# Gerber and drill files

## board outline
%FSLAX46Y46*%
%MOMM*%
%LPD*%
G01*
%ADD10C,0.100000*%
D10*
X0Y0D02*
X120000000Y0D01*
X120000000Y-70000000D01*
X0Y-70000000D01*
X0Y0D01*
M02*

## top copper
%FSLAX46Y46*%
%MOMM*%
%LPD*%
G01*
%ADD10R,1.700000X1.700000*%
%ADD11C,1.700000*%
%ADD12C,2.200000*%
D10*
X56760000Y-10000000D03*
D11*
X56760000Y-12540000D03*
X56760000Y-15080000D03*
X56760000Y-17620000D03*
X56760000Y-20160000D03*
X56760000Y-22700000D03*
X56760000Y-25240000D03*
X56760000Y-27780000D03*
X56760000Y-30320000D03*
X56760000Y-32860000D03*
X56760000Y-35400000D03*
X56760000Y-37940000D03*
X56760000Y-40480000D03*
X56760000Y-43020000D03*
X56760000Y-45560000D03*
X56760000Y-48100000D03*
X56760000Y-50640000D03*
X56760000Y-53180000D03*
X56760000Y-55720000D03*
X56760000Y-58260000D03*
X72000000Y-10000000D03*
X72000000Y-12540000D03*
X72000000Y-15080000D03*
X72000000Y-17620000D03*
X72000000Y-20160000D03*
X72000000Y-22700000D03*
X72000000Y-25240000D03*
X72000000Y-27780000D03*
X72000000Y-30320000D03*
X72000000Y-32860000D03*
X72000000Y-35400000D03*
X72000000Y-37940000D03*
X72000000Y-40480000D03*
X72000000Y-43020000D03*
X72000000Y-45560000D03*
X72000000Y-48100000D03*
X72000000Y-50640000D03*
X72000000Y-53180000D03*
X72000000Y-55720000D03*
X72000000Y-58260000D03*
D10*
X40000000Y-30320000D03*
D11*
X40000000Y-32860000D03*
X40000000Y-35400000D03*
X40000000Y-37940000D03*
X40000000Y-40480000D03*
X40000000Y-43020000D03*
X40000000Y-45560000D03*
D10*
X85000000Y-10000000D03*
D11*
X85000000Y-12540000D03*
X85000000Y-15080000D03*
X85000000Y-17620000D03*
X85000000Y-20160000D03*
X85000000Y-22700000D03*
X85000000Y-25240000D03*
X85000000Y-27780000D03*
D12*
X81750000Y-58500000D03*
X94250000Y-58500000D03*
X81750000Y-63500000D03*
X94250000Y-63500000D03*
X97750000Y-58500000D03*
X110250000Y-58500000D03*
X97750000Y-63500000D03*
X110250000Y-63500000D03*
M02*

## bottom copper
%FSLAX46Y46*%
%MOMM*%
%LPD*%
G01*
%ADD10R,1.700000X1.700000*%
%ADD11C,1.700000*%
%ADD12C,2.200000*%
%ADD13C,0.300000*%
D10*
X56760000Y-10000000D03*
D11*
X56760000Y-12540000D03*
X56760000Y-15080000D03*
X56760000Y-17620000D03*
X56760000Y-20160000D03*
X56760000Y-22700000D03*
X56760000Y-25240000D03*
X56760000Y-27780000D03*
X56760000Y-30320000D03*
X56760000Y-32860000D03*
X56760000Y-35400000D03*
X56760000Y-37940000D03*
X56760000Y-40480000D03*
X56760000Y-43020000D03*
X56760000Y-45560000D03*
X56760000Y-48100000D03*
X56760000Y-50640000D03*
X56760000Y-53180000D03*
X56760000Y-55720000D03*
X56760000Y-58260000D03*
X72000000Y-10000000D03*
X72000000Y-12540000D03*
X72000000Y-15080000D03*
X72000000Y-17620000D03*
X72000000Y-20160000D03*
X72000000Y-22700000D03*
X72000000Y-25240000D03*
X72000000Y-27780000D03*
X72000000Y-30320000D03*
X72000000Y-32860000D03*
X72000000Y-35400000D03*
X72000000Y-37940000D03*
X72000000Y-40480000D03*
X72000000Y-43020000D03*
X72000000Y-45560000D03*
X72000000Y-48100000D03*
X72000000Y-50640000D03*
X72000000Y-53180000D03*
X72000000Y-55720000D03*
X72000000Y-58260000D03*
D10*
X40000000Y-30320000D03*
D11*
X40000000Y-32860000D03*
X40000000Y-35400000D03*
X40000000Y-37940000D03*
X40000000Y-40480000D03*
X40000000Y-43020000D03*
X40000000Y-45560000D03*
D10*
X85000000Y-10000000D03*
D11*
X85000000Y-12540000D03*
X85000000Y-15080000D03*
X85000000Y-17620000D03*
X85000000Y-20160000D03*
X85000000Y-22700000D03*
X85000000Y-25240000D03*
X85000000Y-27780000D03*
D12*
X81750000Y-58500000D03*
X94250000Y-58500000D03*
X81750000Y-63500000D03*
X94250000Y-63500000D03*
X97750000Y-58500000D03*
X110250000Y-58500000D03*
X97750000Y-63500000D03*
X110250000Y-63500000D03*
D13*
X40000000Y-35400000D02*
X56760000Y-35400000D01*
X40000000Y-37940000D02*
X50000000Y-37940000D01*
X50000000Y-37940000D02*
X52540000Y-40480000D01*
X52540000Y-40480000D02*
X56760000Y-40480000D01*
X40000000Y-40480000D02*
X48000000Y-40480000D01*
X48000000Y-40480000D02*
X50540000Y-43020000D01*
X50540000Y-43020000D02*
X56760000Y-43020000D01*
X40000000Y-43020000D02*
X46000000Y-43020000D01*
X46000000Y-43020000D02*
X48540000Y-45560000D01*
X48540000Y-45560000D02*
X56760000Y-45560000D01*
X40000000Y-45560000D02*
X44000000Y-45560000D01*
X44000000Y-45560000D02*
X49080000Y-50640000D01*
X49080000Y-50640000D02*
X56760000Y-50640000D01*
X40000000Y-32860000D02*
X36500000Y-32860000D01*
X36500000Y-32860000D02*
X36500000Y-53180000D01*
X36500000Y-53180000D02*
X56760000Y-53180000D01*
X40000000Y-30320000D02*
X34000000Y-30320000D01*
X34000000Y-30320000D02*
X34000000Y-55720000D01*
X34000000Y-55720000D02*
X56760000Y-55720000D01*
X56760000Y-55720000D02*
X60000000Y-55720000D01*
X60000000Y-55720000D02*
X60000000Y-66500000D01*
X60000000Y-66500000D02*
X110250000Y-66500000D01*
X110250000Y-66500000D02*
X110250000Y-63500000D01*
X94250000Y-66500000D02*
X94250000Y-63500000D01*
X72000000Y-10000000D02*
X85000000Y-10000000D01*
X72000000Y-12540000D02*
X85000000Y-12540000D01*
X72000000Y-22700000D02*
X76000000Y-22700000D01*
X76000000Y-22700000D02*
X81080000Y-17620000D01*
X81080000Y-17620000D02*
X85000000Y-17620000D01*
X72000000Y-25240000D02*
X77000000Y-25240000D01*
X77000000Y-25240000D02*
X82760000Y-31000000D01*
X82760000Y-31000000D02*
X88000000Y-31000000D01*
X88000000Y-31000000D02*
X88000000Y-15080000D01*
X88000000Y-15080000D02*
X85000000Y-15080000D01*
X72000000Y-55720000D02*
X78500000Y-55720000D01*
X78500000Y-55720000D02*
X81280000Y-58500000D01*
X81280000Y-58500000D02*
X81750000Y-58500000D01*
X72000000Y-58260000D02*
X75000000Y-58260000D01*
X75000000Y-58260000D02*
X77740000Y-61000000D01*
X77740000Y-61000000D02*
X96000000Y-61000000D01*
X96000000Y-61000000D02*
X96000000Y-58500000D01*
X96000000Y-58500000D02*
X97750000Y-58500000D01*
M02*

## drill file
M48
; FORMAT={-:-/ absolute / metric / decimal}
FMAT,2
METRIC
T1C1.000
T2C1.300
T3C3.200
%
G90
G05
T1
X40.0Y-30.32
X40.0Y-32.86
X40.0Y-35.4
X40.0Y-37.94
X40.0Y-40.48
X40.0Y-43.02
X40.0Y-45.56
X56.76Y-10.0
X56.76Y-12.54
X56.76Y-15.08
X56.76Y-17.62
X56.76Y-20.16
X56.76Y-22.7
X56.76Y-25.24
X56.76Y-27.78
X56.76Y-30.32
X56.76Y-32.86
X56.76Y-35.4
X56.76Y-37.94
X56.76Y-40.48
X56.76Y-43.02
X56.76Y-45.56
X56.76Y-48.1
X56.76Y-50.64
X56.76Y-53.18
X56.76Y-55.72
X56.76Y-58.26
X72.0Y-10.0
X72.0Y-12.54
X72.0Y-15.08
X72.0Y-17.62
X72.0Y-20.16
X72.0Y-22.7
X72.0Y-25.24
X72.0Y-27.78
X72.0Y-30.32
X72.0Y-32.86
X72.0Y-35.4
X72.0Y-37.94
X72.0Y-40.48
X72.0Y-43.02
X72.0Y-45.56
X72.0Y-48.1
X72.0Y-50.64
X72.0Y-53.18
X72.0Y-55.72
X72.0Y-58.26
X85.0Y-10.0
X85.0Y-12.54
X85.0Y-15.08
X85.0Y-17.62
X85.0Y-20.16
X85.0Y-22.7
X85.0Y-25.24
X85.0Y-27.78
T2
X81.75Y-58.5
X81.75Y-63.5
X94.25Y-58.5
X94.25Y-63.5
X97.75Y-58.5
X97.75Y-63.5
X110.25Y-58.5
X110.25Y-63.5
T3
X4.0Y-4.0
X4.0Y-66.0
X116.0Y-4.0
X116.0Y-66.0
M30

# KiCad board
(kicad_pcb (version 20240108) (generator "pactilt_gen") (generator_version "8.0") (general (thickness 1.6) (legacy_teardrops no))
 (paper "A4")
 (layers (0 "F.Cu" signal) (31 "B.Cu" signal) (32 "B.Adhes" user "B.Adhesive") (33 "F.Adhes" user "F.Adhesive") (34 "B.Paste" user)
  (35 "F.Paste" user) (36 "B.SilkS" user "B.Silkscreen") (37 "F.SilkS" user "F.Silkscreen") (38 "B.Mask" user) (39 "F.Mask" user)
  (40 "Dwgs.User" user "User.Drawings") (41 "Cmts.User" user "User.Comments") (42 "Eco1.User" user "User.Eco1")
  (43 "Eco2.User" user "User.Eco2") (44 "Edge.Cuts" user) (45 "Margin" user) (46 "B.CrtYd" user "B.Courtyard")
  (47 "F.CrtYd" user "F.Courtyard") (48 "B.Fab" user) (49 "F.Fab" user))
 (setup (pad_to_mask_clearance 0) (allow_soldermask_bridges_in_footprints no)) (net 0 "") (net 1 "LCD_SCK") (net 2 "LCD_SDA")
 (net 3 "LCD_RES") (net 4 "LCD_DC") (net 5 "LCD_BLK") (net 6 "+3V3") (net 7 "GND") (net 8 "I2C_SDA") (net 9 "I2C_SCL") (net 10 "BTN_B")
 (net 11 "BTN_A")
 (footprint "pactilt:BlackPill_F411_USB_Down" (layer "F.Cu") (at 56.76 10)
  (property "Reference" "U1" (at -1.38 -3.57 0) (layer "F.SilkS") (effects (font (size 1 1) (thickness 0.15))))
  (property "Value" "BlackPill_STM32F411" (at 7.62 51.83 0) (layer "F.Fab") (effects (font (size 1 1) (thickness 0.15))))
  (pad "1" thru_hole rect (at 0 0) (size 1.7 1.7) (drill 1.0) (layers "*.Cu" "*.Mask"))
  (pad "2" thru_hole circle (at 0 2.54) (size 1.7 1.7) (drill 1.0) (layers "*.Cu" "*.Mask"))
  (pad "3" thru_hole circle (at 0 5.08) (size 1.7 1.7) (drill 1.0) (layers "*.Cu" "*.Mask"))
  (pad "4" thru_hole circle (at 0 7.62) (size 1.7 1.7) (drill 1.0) (layers "*.Cu" "*.Mask"))
  (pad "5" thru_hole circle (at 0 10.16) (size 1.7 1.7) (drill 1.0) (layers "*.Cu" "*.Mask"))
  (pad "6" thru_hole circle (at 0 12.7) (size 1.7 1.7) (drill 1.0) (layers "*.Cu" "*.Mask"))
  (pad "7" thru_hole circle (at 0 15.24) (size 1.7 1.7) (drill 1.0) (layers "*.Cu" "*.Mask"))
  (pad "8" thru_hole circle (at 0 17.78) (size 1.7 1.7) (drill 1.0) (layers "*.Cu" "*.Mask"))
  (pad "9" thru_hole circle (at 0 20.32) (size 1.7 1.7) (drill 1.0) (layers "*.Cu" "*.Mask"))
  (pad "10" thru_hole circle (at 0 22.86) (size 1.7 1.7) (drill 1.0) (layers "*.Cu" "*.Mask"))
  (pad "11" thru_hole circle (at 0 25.4) (size 1.7 1.7) (drill 1.0) (layers "*.Cu" "*.Mask") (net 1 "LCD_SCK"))
  (pad "12" thru_hole circle (at 0 27.94) (size 1.7 1.7) (drill 1.0) (layers "*.Cu" "*.Mask"))
  (pad "13" thru_hole circle (at 0 30.48) (size 1.7 1.7) (drill 1.0) (layers "*.Cu" "*.Mask") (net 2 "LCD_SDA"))
  (pad "14" thru_hole circle (at 0 33.02) (size 1.7 1.7) (drill 1.0) (layers "*.Cu" "*.Mask") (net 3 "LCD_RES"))
  (pad "15" thru_hole circle (at 0 35.56) (size 1.7 1.7) (drill 1.0) (layers "*.Cu" "*.Mask") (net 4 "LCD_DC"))
  (pad "16" thru_hole circle (at 0 38.1) (size 1.7 1.7) (drill 1.0) (layers "*.Cu" "*.Mask"))
  (pad "17" thru_hole circle (at 0 40.64) (size 1.7 1.7) (drill 1.0) (layers "*.Cu" "*.Mask") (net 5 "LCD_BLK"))
  (pad "18" thru_hole circle (at 0 43.18) (size 1.7 1.7) (drill 1.0) (layers "*.Cu" "*.Mask") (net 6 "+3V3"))
  (pad "19" thru_hole circle (at 0 45.72) (size 1.7 1.7) (drill 1.0) (layers "*.Cu" "*.Mask") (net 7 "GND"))
  (pad "20" thru_hole circle (at 0 48.26) (size 1.7 1.7) (drill 1.0) (layers "*.Cu" "*.Mask"))
  (pad "21" thru_hole circle (at 15.24 0) (size 1.7 1.7) (drill 1.0) (layers "*.Cu" "*.Mask") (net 6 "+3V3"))
  (pad "22" thru_hole circle (at 15.24 2.54) (size 1.7 1.7) (drill 1.0) (layers "*.Cu" "*.Mask") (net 7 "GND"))
  (pad "23" thru_hole circle (at 15.24 5.08) (size 1.7 1.7) (drill 1.0) (layers "*.Cu" "*.Mask"))
  (pad "24" thru_hole circle (at 15.24 7.62) (size 1.7 1.7) (drill 1.0) (layers "*.Cu" "*.Mask"))
  (pad "25" thru_hole circle (at 15.24 10.16) (size 1.7 1.7) (drill 1.0) (layers "*.Cu" "*.Mask"))
  (pad "26" thru_hole circle (at 15.24 12.7) (size 1.7 1.7) (drill 1.0) (layers "*.Cu" "*.Mask") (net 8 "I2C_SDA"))
  (pad "27" thru_hole circle (at 15.24 15.24) (size 1.7 1.7) (drill 1.0) (layers "*.Cu" "*.Mask") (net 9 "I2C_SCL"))
  (pad "28" thru_hole circle (at 15.24 17.78) (size 1.7 1.7) (drill 1.0) (layers "*.Cu" "*.Mask"))
  (pad "29" thru_hole circle (at 15.24 20.32) (size 1.7 1.7) (drill 1.0) (layers "*.Cu" "*.Mask"))
  (pad "30" thru_hole circle (at 15.24 22.86) (size 1.7 1.7) (drill 1.0) (layers "*.Cu" "*.Mask"))
  (pad "31" thru_hole circle (at 15.24 25.4) (size 1.7 1.7) (drill 1.0) (layers "*.Cu" "*.Mask"))
  (pad "32" thru_hole circle (at 15.24 27.94) (size 1.7 1.7) (drill 1.0) (layers "*.Cu" "*.Mask"))
  (pad "33" thru_hole circle (at 15.24 30.48) (size 1.7 1.7) (drill 1.0) (layers "*.Cu" "*.Mask"))
  (pad "34" thru_hole circle (at 15.24 33.02) (size 1.7 1.7) (drill 1.0) (layers "*.Cu" "*.Mask"))
  (pad "35" thru_hole circle (at 15.24 35.56) (size 1.7 1.7) (drill 1.0) (layers "*.Cu" "*.Mask"))
  (pad "36" thru_hole circle (at 15.24 38.1) (size 1.7 1.7) (drill 1.0) (layers "*.Cu" "*.Mask"))
  (pad "37" thru_hole circle (at 15.24 40.64) (size 1.7 1.7) (drill 1.0) (layers "*.Cu" "*.Mask"))
  (pad "38" thru_hole circle (at 15.24 43.18) (size 1.7 1.7) (drill 1.0) (layers "*.Cu" "*.Mask"))
  (pad "39" thru_hole circle (at 15.24 45.72) (size 1.7 1.7) (drill 1.0) (layers "*.Cu" "*.Mask") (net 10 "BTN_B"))
  (pad "40" thru_hole circle (at 15.24 48.26) (size 1.7 1.7) (drill 1.0) (layers "*.Cu" "*.Mask") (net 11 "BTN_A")))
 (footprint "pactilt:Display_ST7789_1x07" (layer "F.Cu") (at 40 30.32)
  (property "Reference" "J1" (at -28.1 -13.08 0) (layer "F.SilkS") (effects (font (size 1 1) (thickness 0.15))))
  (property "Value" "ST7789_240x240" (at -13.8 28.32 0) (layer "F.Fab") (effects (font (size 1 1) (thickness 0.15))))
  (pad "1" thru_hole rect (at 0 0) (size 1.7 1.7) (drill 1.0) (layers "*.Cu" "*.Mask") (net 7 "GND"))
  (pad "2" thru_hole circle (at 0 2.54) (size 1.7 1.7) (drill 1.0) (layers "*.Cu" "*.Mask") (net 6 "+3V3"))
  (pad "3" thru_hole circle (at 0 5.08) (size 1.7 1.7) (drill 1.0) (layers "*.Cu" "*.Mask") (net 1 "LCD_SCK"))
  (pad "4" thru_hole circle (at 0 7.62) (size 1.7 1.7) (drill 1.0) (layers "*.Cu" "*.Mask") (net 2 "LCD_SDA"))
  (pad "5" thru_hole circle (at 0 10.16) (size 1.7 1.7) (drill 1.0) (layers "*.Cu" "*.Mask") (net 3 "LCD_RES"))
  (pad "6" thru_hole circle (at 0 12.7) (size 1.7 1.7) (drill 1.0) (layers "*.Cu" "*.Mask") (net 4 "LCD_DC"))
  (pad "7" thru_hole circle (at 0 15.24) (size 1.7 1.7) (drill 1.0) (layers "*.Cu" "*.Mask") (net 5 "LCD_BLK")))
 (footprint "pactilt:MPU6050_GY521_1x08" (layer "F.Cu") (at 85 10)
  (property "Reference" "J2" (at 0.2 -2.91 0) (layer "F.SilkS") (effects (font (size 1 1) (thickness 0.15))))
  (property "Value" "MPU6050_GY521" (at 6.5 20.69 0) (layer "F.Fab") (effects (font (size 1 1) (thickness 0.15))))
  (pad "1" thru_hole rect (at 0 0) (size 1.7 1.7) (drill 1.0) (layers "*.Cu" "*.Mask") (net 6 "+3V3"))
  (pad "2" thru_hole circle (at 0 2.54) (size 1.7 1.7) (drill 1.0) (layers "*.Cu" "*.Mask") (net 7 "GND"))
  (pad "3" thru_hole circle (at 0 5.08) (size 1.7 1.7) (drill 1.0) (layers "*.Cu" "*.Mask") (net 9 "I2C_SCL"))
  (pad "4" thru_hole circle (at 0 7.62) (size 1.7 1.7) (drill 1.0) (layers "*.Cu" "*.Mask") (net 8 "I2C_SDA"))
  (pad "5" thru_hole circle (at 0 10.16) (size 1.7 1.7) (drill 1.0) (layers "*.Cu" "*.Mask"))
  (pad "6" thru_hole circle (at 0 12.7) (size 1.7 1.7) (drill 1.0) (layers "*.Cu" "*.Mask"))
  (pad "7" thru_hole circle (at 0 15.24) (size 1.7 1.7) (drill 1.0) (layers "*.Cu" "*.Mask"))
  (pad "8" thru_hole circle (at 0 17.78) (size 1.7 1.7) (drill 1.0) (layers "*.Cu" "*.Mask")))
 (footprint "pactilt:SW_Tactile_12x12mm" (layer "F.Cu") (at 81.75 58.5)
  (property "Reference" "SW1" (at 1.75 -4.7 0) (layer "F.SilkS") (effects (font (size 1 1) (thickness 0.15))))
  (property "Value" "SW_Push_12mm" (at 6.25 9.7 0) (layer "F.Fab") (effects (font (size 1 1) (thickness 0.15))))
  (pad "1" thru_hole circle (at 0 0) (size 2.2 2.2) (drill 1.3) (layers "*.Cu" "*.Mask") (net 10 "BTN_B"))
  (pad "2" thru_hole circle (at 12.5 0) (size 2.2 2.2) (drill 1.3) (layers "*.Cu" "*.Mask"))
  (pad "3" thru_hole circle (at 0 5) (size 2.2 2.2) (drill 1.3) (layers "*.Cu" "*.Mask"))
  (pad "4" thru_hole circle (at 12.5 5) (size 2.2 2.2) (drill 1.3) (layers "*.Cu" "*.Mask") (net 7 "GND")))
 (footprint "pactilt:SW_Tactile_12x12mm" (layer "F.Cu") (at 97.75 58.5)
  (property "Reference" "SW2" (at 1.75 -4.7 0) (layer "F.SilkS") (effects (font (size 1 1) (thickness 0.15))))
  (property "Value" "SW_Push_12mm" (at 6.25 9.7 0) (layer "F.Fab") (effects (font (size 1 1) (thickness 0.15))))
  (pad "1" thru_hole circle (at 0 0) (size 2.2 2.2) (drill 1.3) (layers "*.Cu" "*.Mask") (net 11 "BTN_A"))
  (pad "2" thru_hole circle (at 12.5 0) (size 2.2 2.2) (drill 1.3) (layers "*.Cu" "*.Mask"))
  (pad "3" thru_hole circle (at 0 5) (size 2.2 2.2) (drill 1.3) (layers "*.Cu" "*.Mask"))
  (pad "4" thru_hole circle (at 12.5 5) (size 2.2 2.2) (drill 1.3) (layers "*.Cu" "*.Mask") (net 7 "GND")))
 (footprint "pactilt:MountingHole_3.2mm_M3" (layer "F.Cu") (at 4 4)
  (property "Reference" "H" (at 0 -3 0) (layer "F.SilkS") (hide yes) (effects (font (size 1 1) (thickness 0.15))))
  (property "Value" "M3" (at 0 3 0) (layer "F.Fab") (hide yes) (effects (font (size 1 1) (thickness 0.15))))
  (pad "" np_thru_hole circle (at 0 0) (size 3.2 3.2) (drill 3.2) (layers "*.Cu" "*.Mask")))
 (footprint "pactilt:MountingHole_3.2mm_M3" (layer "F.Cu") (at 116 4)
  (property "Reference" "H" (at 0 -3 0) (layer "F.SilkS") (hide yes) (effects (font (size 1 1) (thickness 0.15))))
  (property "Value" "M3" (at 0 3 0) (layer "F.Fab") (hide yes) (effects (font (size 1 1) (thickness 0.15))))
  (pad "" np_thru_hole circle (at 0 0) (size 3.2 3.2) (drill 3.2) (layers "*.Cu" "*.Mask")))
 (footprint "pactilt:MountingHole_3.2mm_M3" (layer "F.Cu") (at 4 66)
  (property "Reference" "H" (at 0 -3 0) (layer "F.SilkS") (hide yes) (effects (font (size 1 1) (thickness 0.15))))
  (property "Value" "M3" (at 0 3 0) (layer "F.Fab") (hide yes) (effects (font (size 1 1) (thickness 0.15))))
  (pad "" np_thru_hole circle (at 0 0) (size 3.2 3.2) (drill 3.2) (layers "*.Cu" "*.Mask")))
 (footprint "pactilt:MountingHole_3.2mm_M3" (layer "F.Cu") (at 116 66)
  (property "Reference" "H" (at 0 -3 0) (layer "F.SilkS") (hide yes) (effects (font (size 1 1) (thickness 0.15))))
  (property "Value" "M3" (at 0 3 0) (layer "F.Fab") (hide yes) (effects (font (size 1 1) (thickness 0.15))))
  (pad "" np_thru_hole circle (at 0 0) (size 3.2 3.2) (drill 3.2) (layers "*.Cu" "*.Mask")))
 (segment (start 40 35.4) (end 56.76 35.4) (width 0.3) (layer "B.Cu") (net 1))
 (segment (start 40 37.94) (end 50 37.94) (width 0.3) (layer "B.Cu") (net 2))
 (segment (start 50 37.94) (end 52.54 40.48) (width 0.3) (layer "B.Cu") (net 2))
 (segment (start 52.54 40.48) (end 56.76 40.48) (width 0.3) (layer "B.Cu") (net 2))
 (segment (start 40 40.48) (end 48 40.48) (width 0.3) (layer "B.Cu") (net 3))
 (segment (start 48 40.48) (end 50.54 43.02) (width 0.3) (layer "B.Cu") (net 3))
 (segment (start 50.54 43.02) (end 56.76 43.02) (width 0.3) (layer "B.Cu") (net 3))
 (segment (start 40 43.02) (end 46 43.02) (width 0.3) (layer "B.Cu") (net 4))
 (segment (start 46 43.02) (end 48.54 45.56) (width 0.3) (layer "B.Cu") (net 4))
 (segment (start 48.54 45.56) (end 56.76 45.56) (width 0.3) (layer "B.Cu") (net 4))
 (segment (start 40 45.56) (end 44 45.56) (width 0.3) (layer "B.Cu") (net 5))
 (segment (start 44 45.56) (end 49.08 50.64) (width 0.3) (layer "B.Cu") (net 5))
 (segment (start 49.08 50.64) (end 56.76 50.64) (width 0.3) (layer "B.Cu") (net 5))
 (segment (start 40 32.86) (end 36.5 32.86) (width 0.3) (layer "B.Cu") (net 6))
 (segment (start 36.5 32.86) (end 36.5 53.18) (width 0.3) (layer "B.Cu") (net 6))
 (segment (start 36.5 53.18) (end 56.76 53.18) (width 0.3) (layer "B.Cu") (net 6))
 (segment (start 40 30.32) (end 34 30.32) (width 0.3) (layer "B.Cu") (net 7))
 (segment (start 34 30.32) (end 34 55.72) (width 0.3) (layer "B.Cu") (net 7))
 (segment (start 34 55.72) (end 56.76 55.72) (width 0.3) (layer "B.Cu") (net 7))
 (segment (start 56.76 55.72) (end 60 55.72) (width 0.3) (layer "B.Cu") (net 7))
 (segment (start 60 55.72) (end 60 66.5) (width 0.3) (layer "B.Cu") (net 7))
 (segment (start 60 66.5) (end 110.25 66.5) (width 0.3) (layer "B.Cu") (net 7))
 (segment (start 110.25 66.5) (end 110.25 63.5) (width 0.3) (layer "B.Cu") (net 7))
 (segment (start 94.25 66.5) (end 94.25 63.5) (width 0.3) (layer "B.Cu") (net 7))
 (segment (start 72 10) (end 85 10) (width 0.3) (layer "B.Cu") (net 6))
 (segment (start 72 12.54) (end 85 12.54) (width 0.3) (layer "B.Cu") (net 7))
 (segment (start 72 22.7) (end 76 22.7) (width 0.3) (layer "B.Cu") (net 8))
 (segment (start 76 22.7) (end 81.08 17.62) (width 0.3) (layer "B.Cu") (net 8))
 (segment (start 81.08 17.62) (end 85 17.62) (width 0.3) (layer "B.Cu") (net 8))
 (segment (start 72 25.24) (end 77 25.24) (width 0.3) (layer "B.Cu") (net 9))
 (segment (start 77 25.24) (end 82.76 31) (width 0.3) (layer "B.Cu") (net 9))
 (segment (start 82.76 31) (end 88 31) (width 0.3) (layer "B.Cu") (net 9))
 (segment (start 88 31) (end 88 15.08) (width 0.3) (layer "B.Cu") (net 9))
 (segment (start 88 15.08) (end 85 15.08) (width 0.3) (layer "B.Cu") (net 9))
 (segment (start 72 55.72) (end 78.5 55.72) (width 0.3) (layer "B.Cu") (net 10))
 (segment (start 78.5 55.72) (end 81.28 58.5) (width 0.3) (layer "B.Cu") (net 10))
 (segment (start 81.28 58.5) (end 81.75 58.5) (width 0.3) (layer "B.Cu") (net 10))
 (segment (start 72 58.26) (end 75 58.26) (width 0.3) (layer "B.Cu") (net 11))
 (segment (start 75 58.26) (end 77.74 61) (width 0.3) (layer "B.Cu") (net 11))
 (segment (start 77.74 61) (end 96 61) (width 0.3) (layer "B.Cu") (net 11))
 (segment (start 96 61) (end 96 58.5) (width 0.3) (layer "B.Cu") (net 11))
 (segment (start 96 58.5) (end 97.75 58.5) (width 0.3) (layer "B.Cu") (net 11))
 (gr_rect (start 0 0) (end 120 70) (stroke (width 0.1) (type default)) (fill none) (layer "Edge.Cuts")))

